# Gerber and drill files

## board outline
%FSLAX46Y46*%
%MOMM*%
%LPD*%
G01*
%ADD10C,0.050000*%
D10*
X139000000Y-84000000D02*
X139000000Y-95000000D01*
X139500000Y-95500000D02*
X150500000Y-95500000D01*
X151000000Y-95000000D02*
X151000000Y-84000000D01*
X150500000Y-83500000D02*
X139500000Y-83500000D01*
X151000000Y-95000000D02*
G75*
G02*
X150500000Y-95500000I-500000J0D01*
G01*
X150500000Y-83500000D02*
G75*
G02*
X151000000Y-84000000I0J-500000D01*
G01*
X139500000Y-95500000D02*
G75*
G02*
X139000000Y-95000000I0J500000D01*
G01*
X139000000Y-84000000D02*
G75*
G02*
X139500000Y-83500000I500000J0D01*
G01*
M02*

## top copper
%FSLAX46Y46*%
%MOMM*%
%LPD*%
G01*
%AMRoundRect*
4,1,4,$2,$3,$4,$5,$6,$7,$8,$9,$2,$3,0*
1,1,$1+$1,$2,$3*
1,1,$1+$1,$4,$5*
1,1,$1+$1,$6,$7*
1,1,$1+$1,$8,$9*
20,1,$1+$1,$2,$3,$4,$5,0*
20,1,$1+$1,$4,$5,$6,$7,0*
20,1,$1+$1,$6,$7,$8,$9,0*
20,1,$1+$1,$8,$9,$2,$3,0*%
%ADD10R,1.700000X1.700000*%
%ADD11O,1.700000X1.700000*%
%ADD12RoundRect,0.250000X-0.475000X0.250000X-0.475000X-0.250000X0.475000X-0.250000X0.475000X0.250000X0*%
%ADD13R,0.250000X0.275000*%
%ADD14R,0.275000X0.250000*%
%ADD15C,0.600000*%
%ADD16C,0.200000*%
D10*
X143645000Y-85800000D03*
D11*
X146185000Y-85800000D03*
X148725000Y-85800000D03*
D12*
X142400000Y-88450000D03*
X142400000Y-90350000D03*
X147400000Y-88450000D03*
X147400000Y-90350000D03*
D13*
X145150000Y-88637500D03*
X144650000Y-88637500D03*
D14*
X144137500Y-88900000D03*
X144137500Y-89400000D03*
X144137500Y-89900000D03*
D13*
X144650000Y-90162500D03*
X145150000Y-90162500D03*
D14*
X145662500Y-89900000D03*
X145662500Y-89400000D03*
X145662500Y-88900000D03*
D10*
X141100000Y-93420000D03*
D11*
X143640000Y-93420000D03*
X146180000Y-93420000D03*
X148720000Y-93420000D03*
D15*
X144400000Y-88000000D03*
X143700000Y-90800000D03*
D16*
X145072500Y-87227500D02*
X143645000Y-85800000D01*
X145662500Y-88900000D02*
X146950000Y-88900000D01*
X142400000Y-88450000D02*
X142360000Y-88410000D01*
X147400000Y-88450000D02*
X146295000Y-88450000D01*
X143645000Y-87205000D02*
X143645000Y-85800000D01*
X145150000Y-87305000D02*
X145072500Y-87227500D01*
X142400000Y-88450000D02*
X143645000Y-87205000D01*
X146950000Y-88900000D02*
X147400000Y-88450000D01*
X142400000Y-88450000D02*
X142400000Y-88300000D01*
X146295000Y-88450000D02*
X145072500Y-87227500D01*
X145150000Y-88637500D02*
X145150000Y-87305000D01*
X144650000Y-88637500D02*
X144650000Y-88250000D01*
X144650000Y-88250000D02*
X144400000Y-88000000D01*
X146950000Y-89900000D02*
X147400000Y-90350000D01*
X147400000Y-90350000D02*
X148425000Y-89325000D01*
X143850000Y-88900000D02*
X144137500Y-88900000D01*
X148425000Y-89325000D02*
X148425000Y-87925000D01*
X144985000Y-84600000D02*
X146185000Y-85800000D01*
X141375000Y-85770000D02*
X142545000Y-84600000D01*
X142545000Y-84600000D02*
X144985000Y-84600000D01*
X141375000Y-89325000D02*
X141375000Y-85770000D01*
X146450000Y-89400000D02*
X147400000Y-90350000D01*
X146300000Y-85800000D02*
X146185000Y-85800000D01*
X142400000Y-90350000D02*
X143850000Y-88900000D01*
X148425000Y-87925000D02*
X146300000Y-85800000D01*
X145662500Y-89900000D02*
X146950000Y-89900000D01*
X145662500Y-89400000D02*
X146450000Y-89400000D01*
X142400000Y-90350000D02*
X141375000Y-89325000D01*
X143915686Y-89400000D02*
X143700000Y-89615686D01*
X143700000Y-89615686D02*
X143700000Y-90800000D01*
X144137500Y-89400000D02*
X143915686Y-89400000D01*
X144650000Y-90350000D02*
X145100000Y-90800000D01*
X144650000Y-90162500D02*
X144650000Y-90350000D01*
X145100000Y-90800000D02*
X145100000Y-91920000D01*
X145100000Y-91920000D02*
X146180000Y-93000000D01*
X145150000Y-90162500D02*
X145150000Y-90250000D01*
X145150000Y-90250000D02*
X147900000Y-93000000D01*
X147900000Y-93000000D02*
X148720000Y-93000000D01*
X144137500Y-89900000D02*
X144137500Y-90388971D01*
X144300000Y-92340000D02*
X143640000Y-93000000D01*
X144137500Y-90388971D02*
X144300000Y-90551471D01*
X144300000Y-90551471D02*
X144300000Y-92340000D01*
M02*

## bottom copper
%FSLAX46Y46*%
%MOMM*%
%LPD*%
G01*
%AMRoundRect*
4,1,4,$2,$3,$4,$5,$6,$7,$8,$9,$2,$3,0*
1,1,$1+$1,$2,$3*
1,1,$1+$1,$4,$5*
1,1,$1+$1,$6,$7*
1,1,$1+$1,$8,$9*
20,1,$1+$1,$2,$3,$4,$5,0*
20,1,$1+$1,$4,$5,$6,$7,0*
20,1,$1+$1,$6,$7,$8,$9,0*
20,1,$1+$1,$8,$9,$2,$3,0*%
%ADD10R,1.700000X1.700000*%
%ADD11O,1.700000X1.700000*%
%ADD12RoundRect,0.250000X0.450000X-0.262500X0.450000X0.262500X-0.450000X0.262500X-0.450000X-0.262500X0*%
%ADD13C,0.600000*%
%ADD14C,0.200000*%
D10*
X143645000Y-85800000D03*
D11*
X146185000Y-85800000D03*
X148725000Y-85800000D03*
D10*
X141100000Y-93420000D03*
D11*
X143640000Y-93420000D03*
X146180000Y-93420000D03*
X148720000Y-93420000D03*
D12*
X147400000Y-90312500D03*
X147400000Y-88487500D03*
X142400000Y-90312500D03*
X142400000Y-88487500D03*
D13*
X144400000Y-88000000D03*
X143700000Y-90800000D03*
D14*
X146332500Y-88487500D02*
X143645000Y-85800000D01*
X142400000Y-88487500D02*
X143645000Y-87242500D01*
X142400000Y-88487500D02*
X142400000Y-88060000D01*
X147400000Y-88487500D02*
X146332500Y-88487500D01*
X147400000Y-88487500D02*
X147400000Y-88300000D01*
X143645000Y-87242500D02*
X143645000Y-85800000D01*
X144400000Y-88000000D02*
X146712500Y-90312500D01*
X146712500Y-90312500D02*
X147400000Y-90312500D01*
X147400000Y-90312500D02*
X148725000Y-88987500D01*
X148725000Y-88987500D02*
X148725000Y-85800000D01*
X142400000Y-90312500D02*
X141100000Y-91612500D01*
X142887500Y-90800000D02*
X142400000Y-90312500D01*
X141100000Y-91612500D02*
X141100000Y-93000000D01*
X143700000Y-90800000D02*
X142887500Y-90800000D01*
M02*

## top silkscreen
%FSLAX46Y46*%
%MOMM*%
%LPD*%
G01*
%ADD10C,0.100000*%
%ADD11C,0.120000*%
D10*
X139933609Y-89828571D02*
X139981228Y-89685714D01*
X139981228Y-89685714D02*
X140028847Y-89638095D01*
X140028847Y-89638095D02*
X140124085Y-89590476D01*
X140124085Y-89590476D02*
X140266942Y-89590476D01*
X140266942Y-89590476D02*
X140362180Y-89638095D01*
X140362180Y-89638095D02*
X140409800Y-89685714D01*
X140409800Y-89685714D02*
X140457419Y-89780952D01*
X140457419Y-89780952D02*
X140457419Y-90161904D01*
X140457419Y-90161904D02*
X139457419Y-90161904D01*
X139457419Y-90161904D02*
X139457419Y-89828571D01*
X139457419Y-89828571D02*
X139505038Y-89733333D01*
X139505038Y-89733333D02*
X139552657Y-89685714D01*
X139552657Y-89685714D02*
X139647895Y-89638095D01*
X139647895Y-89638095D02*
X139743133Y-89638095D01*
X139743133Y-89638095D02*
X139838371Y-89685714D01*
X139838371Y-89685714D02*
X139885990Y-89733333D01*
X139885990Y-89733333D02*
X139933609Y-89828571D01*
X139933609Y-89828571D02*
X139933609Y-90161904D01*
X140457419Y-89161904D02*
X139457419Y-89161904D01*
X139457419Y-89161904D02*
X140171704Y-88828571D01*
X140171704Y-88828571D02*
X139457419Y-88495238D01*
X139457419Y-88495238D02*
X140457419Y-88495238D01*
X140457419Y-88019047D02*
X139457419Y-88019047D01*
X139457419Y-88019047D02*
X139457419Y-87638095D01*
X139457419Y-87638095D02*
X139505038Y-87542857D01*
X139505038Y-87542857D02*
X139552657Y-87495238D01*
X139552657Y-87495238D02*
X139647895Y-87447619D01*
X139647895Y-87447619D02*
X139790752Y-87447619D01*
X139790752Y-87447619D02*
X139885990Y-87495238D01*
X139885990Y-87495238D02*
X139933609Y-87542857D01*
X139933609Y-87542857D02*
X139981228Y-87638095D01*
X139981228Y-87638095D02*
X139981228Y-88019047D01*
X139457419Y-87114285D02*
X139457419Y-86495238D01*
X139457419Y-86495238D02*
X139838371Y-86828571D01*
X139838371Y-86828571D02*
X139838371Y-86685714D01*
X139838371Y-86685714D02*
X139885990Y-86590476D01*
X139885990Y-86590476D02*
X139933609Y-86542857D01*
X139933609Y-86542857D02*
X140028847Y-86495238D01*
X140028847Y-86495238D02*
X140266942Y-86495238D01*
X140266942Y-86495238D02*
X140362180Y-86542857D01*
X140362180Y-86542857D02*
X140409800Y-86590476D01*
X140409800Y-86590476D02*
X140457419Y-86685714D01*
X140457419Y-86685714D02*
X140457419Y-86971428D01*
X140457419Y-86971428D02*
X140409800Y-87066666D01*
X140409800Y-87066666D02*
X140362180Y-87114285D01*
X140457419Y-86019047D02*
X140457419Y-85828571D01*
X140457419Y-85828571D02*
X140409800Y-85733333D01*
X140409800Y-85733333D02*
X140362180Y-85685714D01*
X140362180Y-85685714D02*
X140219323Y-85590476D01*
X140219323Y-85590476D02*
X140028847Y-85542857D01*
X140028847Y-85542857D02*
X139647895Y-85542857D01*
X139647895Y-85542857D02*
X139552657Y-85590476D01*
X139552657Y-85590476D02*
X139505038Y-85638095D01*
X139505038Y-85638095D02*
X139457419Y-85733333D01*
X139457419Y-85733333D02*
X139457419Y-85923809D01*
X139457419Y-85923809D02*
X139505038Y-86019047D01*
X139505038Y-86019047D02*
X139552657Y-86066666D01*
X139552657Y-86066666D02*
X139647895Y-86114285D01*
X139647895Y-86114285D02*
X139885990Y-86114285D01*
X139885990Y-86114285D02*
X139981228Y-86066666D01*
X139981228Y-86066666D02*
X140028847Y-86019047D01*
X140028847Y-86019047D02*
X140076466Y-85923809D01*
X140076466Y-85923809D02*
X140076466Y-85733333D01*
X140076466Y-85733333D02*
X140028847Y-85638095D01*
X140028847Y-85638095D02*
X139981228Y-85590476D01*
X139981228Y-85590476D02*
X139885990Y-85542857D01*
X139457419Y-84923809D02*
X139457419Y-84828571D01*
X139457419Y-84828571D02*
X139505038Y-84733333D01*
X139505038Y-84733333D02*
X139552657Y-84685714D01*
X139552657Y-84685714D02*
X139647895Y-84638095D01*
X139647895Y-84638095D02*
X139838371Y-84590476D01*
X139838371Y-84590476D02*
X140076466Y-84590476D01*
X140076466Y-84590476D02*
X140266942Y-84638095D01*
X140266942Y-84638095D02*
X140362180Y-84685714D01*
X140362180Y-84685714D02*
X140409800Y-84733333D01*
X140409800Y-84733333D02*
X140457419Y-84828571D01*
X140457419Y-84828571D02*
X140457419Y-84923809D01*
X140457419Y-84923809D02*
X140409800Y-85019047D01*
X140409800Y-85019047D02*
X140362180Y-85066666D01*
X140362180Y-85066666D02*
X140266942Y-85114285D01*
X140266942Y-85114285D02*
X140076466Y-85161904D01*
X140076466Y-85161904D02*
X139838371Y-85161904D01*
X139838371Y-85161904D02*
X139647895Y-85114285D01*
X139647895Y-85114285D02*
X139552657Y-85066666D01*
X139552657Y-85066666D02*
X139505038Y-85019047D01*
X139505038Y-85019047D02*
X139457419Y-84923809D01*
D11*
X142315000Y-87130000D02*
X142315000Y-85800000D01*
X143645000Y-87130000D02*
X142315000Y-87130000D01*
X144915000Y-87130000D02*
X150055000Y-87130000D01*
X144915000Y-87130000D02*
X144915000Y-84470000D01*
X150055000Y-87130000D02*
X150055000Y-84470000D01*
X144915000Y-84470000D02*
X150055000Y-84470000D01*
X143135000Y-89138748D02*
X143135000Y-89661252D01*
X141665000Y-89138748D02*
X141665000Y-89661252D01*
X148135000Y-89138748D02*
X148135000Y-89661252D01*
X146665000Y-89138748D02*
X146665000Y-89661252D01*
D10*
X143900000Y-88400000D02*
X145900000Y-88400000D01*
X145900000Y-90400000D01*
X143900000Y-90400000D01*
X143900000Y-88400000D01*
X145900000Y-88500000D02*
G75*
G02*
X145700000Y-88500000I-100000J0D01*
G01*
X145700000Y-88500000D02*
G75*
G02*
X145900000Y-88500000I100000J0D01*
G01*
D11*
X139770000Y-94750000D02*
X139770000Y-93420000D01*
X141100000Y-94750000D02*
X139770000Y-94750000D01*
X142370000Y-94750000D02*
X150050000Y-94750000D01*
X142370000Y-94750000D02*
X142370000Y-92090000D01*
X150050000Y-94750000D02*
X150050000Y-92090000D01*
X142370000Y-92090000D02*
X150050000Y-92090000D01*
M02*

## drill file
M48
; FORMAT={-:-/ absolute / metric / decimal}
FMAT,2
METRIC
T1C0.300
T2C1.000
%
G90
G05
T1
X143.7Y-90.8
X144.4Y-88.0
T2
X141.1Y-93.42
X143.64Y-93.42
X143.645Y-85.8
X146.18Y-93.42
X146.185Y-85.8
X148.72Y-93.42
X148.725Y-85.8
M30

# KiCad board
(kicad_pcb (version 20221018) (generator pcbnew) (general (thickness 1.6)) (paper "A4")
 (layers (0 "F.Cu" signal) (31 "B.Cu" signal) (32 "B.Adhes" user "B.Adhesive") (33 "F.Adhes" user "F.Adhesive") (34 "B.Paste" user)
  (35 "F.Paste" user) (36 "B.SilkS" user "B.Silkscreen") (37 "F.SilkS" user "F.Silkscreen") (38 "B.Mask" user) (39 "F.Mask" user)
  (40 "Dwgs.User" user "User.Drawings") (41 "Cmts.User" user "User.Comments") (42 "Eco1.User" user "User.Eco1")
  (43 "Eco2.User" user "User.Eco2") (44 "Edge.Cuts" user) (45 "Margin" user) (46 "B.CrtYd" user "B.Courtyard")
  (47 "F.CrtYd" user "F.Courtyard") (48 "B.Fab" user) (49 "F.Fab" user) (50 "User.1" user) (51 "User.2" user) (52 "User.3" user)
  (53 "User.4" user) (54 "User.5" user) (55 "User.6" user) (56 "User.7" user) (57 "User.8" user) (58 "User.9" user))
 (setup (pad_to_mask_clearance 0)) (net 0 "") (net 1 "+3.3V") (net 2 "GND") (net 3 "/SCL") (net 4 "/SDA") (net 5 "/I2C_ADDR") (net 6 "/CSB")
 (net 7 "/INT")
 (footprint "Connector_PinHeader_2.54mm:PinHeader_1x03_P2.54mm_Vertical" (layer "F.Cu") (at 143.645 85.8 90)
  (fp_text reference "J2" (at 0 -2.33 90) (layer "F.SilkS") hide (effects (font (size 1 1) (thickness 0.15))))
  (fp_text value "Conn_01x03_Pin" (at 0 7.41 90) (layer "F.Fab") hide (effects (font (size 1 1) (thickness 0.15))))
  (fp_line (start -1.33 -1.33) (end 0 -1.33) (stroke (width 0.12) (type solid)) (layer "F.SilkS"))
  (fp_line (start -1.33 0) (end -1.33 -1.33) (stroke (width 0.12) (type solid)) (layer "F.SilkS"))
  (fp_line (start -1.33 1.27) (end -1.33 6.41) (stroke (width 0.12) (type solid)) (layer "F.SilkS"))
  (fp_line (start -1.33 1.27) (end 1.33 1.27) (stroke (width 0.12) (type solid)) (layer "F.SilkS"))
  (fp_line (start -1.33 6.41) (end 1.33 6.41) (stroke (width 0.12) (type solid)) (layer "F.SilkS"))
  (fp_line (start 1.33 1.27) (end 1.33 6.41) (stroke (width 0.12) (type solid)) (layer "F.SilkS"))
  (pad "1" thru_hole rect (at 0 0 90) (size 1.7 1.7) (drill 1) (layers "*.Cu" "*.Mask") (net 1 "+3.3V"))
  (pad "2" thru_hole oval (at 0 2.54 90) (size 1.7 1.7) (drill 1) (layers "*.Cu" "*.Mask") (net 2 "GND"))
  (pad "3" thru_hole oval (at 0 5.08 90) (size 1.7 1.7) (drill 1) (layers "*.Cu" "*.Mask") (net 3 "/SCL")))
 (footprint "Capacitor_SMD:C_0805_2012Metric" (layer "F.Cu") (at 142.4 89.4 -90)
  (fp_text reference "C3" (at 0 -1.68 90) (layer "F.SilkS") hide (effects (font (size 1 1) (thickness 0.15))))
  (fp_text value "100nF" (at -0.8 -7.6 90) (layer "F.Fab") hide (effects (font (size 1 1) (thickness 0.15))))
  (fp_line (start -0.261252 -0.735) (end 0.261252 -0.735) (stroke (width 0.12) (type solid)) (layer "F.SilkS"))
  (fp_line (start -0.261252 0.735) (end 0.261252 0.735) (stroke (width 0.12) (type solid)) (layer "F.SilkS"))
  (pad "1" smd roundrect (at -0.95 0 270) (size 1 1.45) (layers "F.Cu" "F.Paste" "F.Mask") (roundrect_rratio 0.25) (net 1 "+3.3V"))
  (pad "2" smd roundrect (at 0.95 0 270) (size 1 1.45) (layers "F.Cu" "F.Paste" "F.Mask") (roundrect_rratio 0.25) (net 2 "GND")))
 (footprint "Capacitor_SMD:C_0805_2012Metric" (layer "F.Cu") (at 147.4 89.4 -90)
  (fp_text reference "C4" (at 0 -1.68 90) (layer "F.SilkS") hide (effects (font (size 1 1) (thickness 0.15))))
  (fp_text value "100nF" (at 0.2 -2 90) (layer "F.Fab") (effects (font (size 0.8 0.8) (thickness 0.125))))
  (fp_line (start -0.261252 -0.735) (end 0.261252 -0.735) (stroke (width 0.12) (type solid)) (layer "F.SilkS"))
  (fp_line (start -0.261252 0.735) (end 0.261252 0.735) (stroke (width 0.12) (type solid)) (layer "F.SilkS"))
  (pad "1" smd roundrect (at -0.95 0 270) (size 1 1.45) (layers "F.Cu" "F.Paste" "F.Mask") (roundrect_rratio 0.25) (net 1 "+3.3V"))
  (pad "2" smd roundrect (at 0.95 0 270) (size 1 1.45) (layers "F.Cu" "F.Paste" "F.Mask") (roundrect_rratio 0.25) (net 2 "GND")))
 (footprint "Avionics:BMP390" (layer "F.Cu") (at 144.9 89.4)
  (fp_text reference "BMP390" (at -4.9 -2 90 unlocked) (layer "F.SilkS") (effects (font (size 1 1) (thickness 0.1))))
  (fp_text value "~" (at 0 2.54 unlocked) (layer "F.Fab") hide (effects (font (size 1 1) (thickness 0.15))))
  (fp_rect (start -1 -1) (end 1 1) (stroke (width 0.1) (type default)) (fill none) (layer "F.SilkS"))
  (fp_circle (center 0.9 -0.9) (end 1 -0.9) (stroke (width 0.1) (type default)) (fill none) (layer "F.SilkS"))
  (pad "1" smd rect (at 0.25 -0.7625) (size 0.25 0.275) (layers "F.Cu" "F.Paste" "F.Mask") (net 1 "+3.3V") (thermal_bridge_angle 45))
  (pad "2" smd rect (at -0.25 -0.7625) (size 0.25 0.275) (layers "F.Cu" "F.Paste" "F.Mask") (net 3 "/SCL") (thermal_bridge_angle 45))
  (pad "3" smd rect (at -0.7625 -0.5 90) (size 0.25 0.275) (layers "F.Cu" "F.Paste" "F.Mask") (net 2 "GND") (thermal_bridge_angle 45))
  (pad "4" smd rect (at -0.7625 0 90) (size 0.25 0.275) (layers "F.Cu" "F.Paste" "F.Mask") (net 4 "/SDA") (thermal_bridge_angle 45))
  (pad "5" smd rect (at -0.7625 0.5 90) (size 0.25 0.275) (layers "F.Cu" "F.Paste" "F.Mask") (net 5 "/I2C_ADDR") (thermal_bridge_angle 45))
  (pad "6" smd rect (at -0.25 0.7625) (size 0.25 0.275) (layers "F.Cu" "F.Paste" "F.Mask") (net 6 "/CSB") (thermal_bridge_angle 45))
  (pad "7" smd rect (at 0.25 0.7625) (size 0.25 0.275) (layers "F.Cu" "F.Paste" "F.Mask") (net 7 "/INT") (thermal_bridge_angle 45))
  (pad "8" smd rect (at 0.7625 0.5 90) (size 0.25 0.275) (layers "F.Cu" "F.Paste" "F.Mask") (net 2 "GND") (thermal_bridge_angle 45))
  (pad "9" smd rect (at 0.7625 0 90) (size 0.25 0.275) (layers "F.Cu" "F.Paste" "F.Mask") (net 2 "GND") (thermal_bridge_angle 45))
  (pad "10" smd rect (at 0.7625 -0.5 90) (size 0.25 0.275) (layers "F.Cu" "F.Paste" "F.Mask") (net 1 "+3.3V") (thermal_bridge_angle 45)))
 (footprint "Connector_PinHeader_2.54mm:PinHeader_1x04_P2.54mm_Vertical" (layer "F.Cu") (at 141.1 93.42 90)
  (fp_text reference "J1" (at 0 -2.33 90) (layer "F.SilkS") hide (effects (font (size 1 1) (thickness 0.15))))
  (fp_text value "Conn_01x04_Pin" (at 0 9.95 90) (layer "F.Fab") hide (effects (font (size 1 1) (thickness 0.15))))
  (fp_line (start -1.33 -1.33) (end 0 -1.33) (stroke (width 0.12) (type solid)) (layer "F.SilkS"))
  (fp_line (start -1.33 0) (end -1.33 -1.33) (stroke (width 0.12) (type solid)) (layer "F.SilkS"))
  (fp_line (start -1.33 1.27) (end -1.33 8.95) (stroke (width 0.12) (type solid)) (layer "F.SilkS"))
  (fp_line (start -1.33 1.27) (end 1.33 1.27) (stroke (width 0.12) (type solid)) (layer "F.SilkS"))
  (fp_line (start -1.33 8.95) (end 1.33 8.95) (stroke (width 0.12) (type solid)) (layer "F.SilkS"))
  (fp_line (start 1.33 1.27) (end 1.33 8.95) (stroke (width 0.12) (type solid)) (layer "F.SilkS"))
  (pad "1" thru_hole rect (at 0 0 90) (size 1.7 1.7) (drill 1) (layers "*.Cu" "*.Mask") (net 4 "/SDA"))
  (pad "2" thru_hole oval (at 0 2.54 90) (size 1.7 1.7) (drill 1) (layers "*.Cu" "*.Mask") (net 5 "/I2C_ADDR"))
  (pad "3" thru_hole oval (at 0 5.08 90) (size 1.7 1.7) (drill 1) (layers "*.Cu" "*.Mask") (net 6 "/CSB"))
  (pad "4" thru_hole oval (at 0 7.62 90) (size 1.7 1.7) (drill 1) (layers "*.Cu" "*.Mask") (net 7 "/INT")))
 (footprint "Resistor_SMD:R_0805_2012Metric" (layer "B.Cu") (at 147.4 89.4 90)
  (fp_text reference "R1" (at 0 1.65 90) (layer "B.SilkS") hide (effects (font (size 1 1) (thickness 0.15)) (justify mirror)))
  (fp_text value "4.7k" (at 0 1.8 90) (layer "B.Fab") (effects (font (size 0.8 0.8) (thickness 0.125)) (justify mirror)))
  (pad "1" smd roundrect (at -0.9125 0 90) (size 1.025 1.4) (layers "B.Cu" "B.Paste" "B.Mask") (roundrect_rratio 0.243902439) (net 3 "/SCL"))
  (pad "2" smd roundrect (at 0.9125 0 90) (size 1.025 1.4) (layers "B.Cu" "B.Paste" "B.Mask") (roundrect_rratio 0.243902439) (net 1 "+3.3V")))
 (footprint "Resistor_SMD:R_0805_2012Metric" (layer "B.Cu") (at 142.4 89.4 90)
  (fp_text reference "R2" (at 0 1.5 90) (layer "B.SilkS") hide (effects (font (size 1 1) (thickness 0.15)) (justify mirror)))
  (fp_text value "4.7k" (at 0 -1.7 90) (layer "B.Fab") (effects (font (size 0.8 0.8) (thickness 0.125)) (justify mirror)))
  (pad "1" smd roundrect (at -0.9125 0 90) (size 1.025 1.4) (layers "B.Cu" "B.Paste" "B.Mask") (roundrect_rratio 0.243902439) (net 4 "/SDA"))
  (pad "2" smd roundrect (at 0.9125 0 90) (size 1.025 1.4) (layers "B.Cu" "B.Paste" "B.Mask") (roundrect_rratio 0.243902439) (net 1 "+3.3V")))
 (gr_line (start 139 84) (end 139 95) (stroke (width 0.05) (type default)) (layer "Edge.Cuts"))
 (gr_line (start 139.5 95.5) (end 150.5 95.5) (stroke (width 0.05) (type default)) (layer "Edge.Cuts"))
 (gr_line (start 151 95) (end 151 84) (stroke (width 0.05) (type default)) (layer "Edge.Cuts"))
 (gr_line (start 150.5 83.5) (end 139.5 83.5) (stroke (width 0.05) (type default)) (layer "Edge.Cuts"))
 (gr_arc (start 151 95) (mid 150.853553 95.353553) (end 150.5 95.5) (stroke (width 0.05) (type default)) (layer "Edge.Cuts"))
 (gr_arc (start 150.5 83.5) (mid 150.853553 83.646447) (end 151 84) (stroke (width 0.05) (type default)) (layer "Edge.Cuts"))
 (gr_arc (start 139.5 95.5) (mid 139.146447 95.353553) (end 139 95) (stroke (width 0.05) (type default)) (layer "Edge.Cuts"))
 (gr_arc (start 139 84) (mid 139.146447 83.646447) (end 139.5 83.5) (stroke (width 0.05) (type default)) (layer "Edge.Cuts"))
 (segment (start 145.0725 87.2275) (end 143.645 85.8) (width 0.2) (layer "F.Cu") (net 1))
 (segment (start 145.6625 88.9) (end 146.95 88.9) (width 0.2) (layer "F.Cu") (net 1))
 (segment (start 142.4 88.45) (end 142.36 88.41) (width 0.2) (layer "F.Cu") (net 1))
 (segment (start 147.4 88.45) (end 146.295 88.45) (width 0.2) (layer "F.Cu") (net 1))
 (segment (start 143.645 87.205) (end 143.645 85.8) (width 0.2) (layer "F.Cu") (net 1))
 (segment (start 145.15 87.305) (end 145.0725 87.2275) (width 0.2) (layer "F.Cu") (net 1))
 (segment (start 142.4 88.45) (end 143.645 87.205) (width 0.2) (layer "F.Cu") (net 1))
 (segment (start 146.95 88.9) (end 147.4 88.45) (width 0.2) (layer "F.Cu") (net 1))
 (segment (start 142.4 88.45) (end 142.4 88.3) (width 0.2) (layer "F.Cu") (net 1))
 (segment (start 146.295 88.45) (end 145.0725 87.2275) (width 0.2) (layer "F.Cu") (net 1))
 (segment (start 145.15 88.6375) (end 145.15 87.305) (width 0.2) (layer "F.Cu") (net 1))
 (segment (start 146.3325 88.4875) (end 143.645 85.8) (width 0.2) (layer "B.Cu") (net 1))
 (segment (start 142.4 88.4875) (end 143.645 87.2425) (width 0.2) (layer "B.Cu") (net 1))
 (segment (start 142.4 88.4875) (end 142.4 88.06) (width 0.2) (layer "B.Cu") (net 1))
 (segment (start 147.4 88.4875) (end 146.3325 88.4875) (width 0.2) (layer "B.Cu") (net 1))
 (segment (start 147.4 88.4875) (end 147.4 88.3) (width 0.2) (layer "B.Cu") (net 1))
 (segment (start 143.645 87.2425) (end 143.645 85.8) (width 0.2) (layer "B.Cu") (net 1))
 (segment (start 144.65 88.6375) (end 144.65 88.25) (width 0.2) (layer "F.Cu") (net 3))
 (segment (start 144.65 88.25) (end 144.4 88) (width 0.2) (layer "F.Cu") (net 3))
 (via (at 144.4 88) (size 0.6) (drill 0.3) (layers "F.Cu" "B.Cu") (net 3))
 (segment (start 144.4 88) (end 146.7125 90.3125) (width 0.2) (layer "B.Cu") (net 3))
 (segment (start 146.7125 90.3125) (end 147.4 90.3125) (width 0.2) (layer "B.Cu") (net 3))
 (segment (start 147.4 90.3125) (end 148.725 88.9875) (width 0.2) (layer "B.Cu") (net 3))
 (segment (start 148.725 88.9875) (end 148.725 85.8) (width 0.2) (layer "B.Cu") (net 3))
 (segment (start 146.95 89.9) (end 147.4 90.35) (width 0.2) (layer "F.Cu") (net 2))
 (segment (start 147.4 90.35) (end 148.425 89.325) (width 0.2) (layer "F.Cu") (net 2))
 (segment (start 143.85 88.9) (end 144.1375 88.9) (width 0.2) (layer "F.Cu") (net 2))
 (segment (start 148.425 89.325) (end 148.425 87.925) (width 0.2) (layer "F.Cu") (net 2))
 (segment (start 144.985 84.6) (end 146.185 85.8) (width 0.2) (layer "F.Cu") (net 2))
 (segment (start 141.375 85.77) (end 142.545 84.6) (width 0.2) (layer "F.Cu") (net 2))
 (segment (start 142.545 84.6) (end 144.985 84.6) (width 0.2) (layer "F.Cu") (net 2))
 (segment (start 141.375 89.325) (end 141.375 85.77) (width 0.2) (layer "F.Cu") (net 2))
 (segment (start 146.45 89.4) (end 147.4 90.35) (width 0.2) (layer "F.Cu") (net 2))
 (segment (start 146.3 85.8) (end 146.185 85.8) (width 0.2) (layer "F.Cu") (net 2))
 (segment (start 142.4 90.35) (end 143.85 88.9) (width 0.2) (layer "F.Cu") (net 2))
 (segment (start 148.425 87.925) (end 146.3 85.8) (width 0.2) (layer "F.Cu") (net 2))
 (segment (start 145.6625 89.9) (end 146.95 89.9) (width 0.2) (layer "F.Cu") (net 2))
 (segment (start 145.6625 89.4) (end 146.45 89.4) (width 0.2) (layer "F.Cu") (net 2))
 (segment (start 142.4 90.35) (end 141.375 89.325) (width 0.2) (layer "F.Cu") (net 2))
 (segment (start 143.915686 89.4) (end 143.7 89.615686) (width 0.2) (layer "F.Cu") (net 4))
 (segment (start 143.7 89.615686) (end 143.7 90.8) (width 0.2) (layer "F.Cu") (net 4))
 (segment (start 144.1375 89.4) (end 143.915686 89.4) (width 0.2) (layer "F.Cu") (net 4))
 (via (at 143.7 90.8) (size 0.6) (drill 0.3) (layers "F.Cu" "B.Cu") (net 4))
 (segment (start 142.4 90.3125) (end 141.1 91.6125) (width 0.2) (layer "B.Cu") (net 4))
 (segment (start 142.8875 90.8) (end 142.4 90.3125) (width 0.2) (layer "B.Cu") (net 4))
 (segment (start 141.1 91.6125) (end 141.1 93) (width 0.2) (layer "B.Cu") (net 4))
 (segment (start 143.7 90.8) (end 142.8875 90.8) (width 0.2) (layer "B.Cu") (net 4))
 (segment (start 144.65 90.35) (end 145.1 90.8) (width 0.2) (layer "F.Cu") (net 6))
 (segment (start 144.65 90.1625) (end 144.65 90.35) (width 0.2) (layer "F.Cu") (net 6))
 (segment (start 145.1 90.8) (end 145.1 91.92) (width 0.2) (layer "F.Cu") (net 6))
 (segment (start 145.1 91.92) (end 146.18 93) (width 0.2) (layer "F.Cu") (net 6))
 (segment (start 145.15 90.1625) (end 145.15 90.25) (width 0.2) (layer "F.Cu") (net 7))
 (segment (start 145.15 90.25) (end 147.9 93) (width 0.2) (layer "F.Cu") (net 7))
 (segment (start 147.9 93) (end 148.72 93) (width 0.2) (layer "F.Cu") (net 7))
 (segment (start 144.1375 89.9) (end 144.1375 90.388971) (width 0.2) (layer "F.Cu") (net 5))
 (segment (start 144.3 92.34) (end 143.64 93) (width 0.2) (layer "F.Cu") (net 5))
 (segment (start 144.1375 90.388971) (end 144.3 90.551471) (width 0.2) (layer "F.Cu") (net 5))
 (segment (start 144.3 90.551471) (end 144.3 92.34) (width 0.2) (layer "F.Cu") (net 5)))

